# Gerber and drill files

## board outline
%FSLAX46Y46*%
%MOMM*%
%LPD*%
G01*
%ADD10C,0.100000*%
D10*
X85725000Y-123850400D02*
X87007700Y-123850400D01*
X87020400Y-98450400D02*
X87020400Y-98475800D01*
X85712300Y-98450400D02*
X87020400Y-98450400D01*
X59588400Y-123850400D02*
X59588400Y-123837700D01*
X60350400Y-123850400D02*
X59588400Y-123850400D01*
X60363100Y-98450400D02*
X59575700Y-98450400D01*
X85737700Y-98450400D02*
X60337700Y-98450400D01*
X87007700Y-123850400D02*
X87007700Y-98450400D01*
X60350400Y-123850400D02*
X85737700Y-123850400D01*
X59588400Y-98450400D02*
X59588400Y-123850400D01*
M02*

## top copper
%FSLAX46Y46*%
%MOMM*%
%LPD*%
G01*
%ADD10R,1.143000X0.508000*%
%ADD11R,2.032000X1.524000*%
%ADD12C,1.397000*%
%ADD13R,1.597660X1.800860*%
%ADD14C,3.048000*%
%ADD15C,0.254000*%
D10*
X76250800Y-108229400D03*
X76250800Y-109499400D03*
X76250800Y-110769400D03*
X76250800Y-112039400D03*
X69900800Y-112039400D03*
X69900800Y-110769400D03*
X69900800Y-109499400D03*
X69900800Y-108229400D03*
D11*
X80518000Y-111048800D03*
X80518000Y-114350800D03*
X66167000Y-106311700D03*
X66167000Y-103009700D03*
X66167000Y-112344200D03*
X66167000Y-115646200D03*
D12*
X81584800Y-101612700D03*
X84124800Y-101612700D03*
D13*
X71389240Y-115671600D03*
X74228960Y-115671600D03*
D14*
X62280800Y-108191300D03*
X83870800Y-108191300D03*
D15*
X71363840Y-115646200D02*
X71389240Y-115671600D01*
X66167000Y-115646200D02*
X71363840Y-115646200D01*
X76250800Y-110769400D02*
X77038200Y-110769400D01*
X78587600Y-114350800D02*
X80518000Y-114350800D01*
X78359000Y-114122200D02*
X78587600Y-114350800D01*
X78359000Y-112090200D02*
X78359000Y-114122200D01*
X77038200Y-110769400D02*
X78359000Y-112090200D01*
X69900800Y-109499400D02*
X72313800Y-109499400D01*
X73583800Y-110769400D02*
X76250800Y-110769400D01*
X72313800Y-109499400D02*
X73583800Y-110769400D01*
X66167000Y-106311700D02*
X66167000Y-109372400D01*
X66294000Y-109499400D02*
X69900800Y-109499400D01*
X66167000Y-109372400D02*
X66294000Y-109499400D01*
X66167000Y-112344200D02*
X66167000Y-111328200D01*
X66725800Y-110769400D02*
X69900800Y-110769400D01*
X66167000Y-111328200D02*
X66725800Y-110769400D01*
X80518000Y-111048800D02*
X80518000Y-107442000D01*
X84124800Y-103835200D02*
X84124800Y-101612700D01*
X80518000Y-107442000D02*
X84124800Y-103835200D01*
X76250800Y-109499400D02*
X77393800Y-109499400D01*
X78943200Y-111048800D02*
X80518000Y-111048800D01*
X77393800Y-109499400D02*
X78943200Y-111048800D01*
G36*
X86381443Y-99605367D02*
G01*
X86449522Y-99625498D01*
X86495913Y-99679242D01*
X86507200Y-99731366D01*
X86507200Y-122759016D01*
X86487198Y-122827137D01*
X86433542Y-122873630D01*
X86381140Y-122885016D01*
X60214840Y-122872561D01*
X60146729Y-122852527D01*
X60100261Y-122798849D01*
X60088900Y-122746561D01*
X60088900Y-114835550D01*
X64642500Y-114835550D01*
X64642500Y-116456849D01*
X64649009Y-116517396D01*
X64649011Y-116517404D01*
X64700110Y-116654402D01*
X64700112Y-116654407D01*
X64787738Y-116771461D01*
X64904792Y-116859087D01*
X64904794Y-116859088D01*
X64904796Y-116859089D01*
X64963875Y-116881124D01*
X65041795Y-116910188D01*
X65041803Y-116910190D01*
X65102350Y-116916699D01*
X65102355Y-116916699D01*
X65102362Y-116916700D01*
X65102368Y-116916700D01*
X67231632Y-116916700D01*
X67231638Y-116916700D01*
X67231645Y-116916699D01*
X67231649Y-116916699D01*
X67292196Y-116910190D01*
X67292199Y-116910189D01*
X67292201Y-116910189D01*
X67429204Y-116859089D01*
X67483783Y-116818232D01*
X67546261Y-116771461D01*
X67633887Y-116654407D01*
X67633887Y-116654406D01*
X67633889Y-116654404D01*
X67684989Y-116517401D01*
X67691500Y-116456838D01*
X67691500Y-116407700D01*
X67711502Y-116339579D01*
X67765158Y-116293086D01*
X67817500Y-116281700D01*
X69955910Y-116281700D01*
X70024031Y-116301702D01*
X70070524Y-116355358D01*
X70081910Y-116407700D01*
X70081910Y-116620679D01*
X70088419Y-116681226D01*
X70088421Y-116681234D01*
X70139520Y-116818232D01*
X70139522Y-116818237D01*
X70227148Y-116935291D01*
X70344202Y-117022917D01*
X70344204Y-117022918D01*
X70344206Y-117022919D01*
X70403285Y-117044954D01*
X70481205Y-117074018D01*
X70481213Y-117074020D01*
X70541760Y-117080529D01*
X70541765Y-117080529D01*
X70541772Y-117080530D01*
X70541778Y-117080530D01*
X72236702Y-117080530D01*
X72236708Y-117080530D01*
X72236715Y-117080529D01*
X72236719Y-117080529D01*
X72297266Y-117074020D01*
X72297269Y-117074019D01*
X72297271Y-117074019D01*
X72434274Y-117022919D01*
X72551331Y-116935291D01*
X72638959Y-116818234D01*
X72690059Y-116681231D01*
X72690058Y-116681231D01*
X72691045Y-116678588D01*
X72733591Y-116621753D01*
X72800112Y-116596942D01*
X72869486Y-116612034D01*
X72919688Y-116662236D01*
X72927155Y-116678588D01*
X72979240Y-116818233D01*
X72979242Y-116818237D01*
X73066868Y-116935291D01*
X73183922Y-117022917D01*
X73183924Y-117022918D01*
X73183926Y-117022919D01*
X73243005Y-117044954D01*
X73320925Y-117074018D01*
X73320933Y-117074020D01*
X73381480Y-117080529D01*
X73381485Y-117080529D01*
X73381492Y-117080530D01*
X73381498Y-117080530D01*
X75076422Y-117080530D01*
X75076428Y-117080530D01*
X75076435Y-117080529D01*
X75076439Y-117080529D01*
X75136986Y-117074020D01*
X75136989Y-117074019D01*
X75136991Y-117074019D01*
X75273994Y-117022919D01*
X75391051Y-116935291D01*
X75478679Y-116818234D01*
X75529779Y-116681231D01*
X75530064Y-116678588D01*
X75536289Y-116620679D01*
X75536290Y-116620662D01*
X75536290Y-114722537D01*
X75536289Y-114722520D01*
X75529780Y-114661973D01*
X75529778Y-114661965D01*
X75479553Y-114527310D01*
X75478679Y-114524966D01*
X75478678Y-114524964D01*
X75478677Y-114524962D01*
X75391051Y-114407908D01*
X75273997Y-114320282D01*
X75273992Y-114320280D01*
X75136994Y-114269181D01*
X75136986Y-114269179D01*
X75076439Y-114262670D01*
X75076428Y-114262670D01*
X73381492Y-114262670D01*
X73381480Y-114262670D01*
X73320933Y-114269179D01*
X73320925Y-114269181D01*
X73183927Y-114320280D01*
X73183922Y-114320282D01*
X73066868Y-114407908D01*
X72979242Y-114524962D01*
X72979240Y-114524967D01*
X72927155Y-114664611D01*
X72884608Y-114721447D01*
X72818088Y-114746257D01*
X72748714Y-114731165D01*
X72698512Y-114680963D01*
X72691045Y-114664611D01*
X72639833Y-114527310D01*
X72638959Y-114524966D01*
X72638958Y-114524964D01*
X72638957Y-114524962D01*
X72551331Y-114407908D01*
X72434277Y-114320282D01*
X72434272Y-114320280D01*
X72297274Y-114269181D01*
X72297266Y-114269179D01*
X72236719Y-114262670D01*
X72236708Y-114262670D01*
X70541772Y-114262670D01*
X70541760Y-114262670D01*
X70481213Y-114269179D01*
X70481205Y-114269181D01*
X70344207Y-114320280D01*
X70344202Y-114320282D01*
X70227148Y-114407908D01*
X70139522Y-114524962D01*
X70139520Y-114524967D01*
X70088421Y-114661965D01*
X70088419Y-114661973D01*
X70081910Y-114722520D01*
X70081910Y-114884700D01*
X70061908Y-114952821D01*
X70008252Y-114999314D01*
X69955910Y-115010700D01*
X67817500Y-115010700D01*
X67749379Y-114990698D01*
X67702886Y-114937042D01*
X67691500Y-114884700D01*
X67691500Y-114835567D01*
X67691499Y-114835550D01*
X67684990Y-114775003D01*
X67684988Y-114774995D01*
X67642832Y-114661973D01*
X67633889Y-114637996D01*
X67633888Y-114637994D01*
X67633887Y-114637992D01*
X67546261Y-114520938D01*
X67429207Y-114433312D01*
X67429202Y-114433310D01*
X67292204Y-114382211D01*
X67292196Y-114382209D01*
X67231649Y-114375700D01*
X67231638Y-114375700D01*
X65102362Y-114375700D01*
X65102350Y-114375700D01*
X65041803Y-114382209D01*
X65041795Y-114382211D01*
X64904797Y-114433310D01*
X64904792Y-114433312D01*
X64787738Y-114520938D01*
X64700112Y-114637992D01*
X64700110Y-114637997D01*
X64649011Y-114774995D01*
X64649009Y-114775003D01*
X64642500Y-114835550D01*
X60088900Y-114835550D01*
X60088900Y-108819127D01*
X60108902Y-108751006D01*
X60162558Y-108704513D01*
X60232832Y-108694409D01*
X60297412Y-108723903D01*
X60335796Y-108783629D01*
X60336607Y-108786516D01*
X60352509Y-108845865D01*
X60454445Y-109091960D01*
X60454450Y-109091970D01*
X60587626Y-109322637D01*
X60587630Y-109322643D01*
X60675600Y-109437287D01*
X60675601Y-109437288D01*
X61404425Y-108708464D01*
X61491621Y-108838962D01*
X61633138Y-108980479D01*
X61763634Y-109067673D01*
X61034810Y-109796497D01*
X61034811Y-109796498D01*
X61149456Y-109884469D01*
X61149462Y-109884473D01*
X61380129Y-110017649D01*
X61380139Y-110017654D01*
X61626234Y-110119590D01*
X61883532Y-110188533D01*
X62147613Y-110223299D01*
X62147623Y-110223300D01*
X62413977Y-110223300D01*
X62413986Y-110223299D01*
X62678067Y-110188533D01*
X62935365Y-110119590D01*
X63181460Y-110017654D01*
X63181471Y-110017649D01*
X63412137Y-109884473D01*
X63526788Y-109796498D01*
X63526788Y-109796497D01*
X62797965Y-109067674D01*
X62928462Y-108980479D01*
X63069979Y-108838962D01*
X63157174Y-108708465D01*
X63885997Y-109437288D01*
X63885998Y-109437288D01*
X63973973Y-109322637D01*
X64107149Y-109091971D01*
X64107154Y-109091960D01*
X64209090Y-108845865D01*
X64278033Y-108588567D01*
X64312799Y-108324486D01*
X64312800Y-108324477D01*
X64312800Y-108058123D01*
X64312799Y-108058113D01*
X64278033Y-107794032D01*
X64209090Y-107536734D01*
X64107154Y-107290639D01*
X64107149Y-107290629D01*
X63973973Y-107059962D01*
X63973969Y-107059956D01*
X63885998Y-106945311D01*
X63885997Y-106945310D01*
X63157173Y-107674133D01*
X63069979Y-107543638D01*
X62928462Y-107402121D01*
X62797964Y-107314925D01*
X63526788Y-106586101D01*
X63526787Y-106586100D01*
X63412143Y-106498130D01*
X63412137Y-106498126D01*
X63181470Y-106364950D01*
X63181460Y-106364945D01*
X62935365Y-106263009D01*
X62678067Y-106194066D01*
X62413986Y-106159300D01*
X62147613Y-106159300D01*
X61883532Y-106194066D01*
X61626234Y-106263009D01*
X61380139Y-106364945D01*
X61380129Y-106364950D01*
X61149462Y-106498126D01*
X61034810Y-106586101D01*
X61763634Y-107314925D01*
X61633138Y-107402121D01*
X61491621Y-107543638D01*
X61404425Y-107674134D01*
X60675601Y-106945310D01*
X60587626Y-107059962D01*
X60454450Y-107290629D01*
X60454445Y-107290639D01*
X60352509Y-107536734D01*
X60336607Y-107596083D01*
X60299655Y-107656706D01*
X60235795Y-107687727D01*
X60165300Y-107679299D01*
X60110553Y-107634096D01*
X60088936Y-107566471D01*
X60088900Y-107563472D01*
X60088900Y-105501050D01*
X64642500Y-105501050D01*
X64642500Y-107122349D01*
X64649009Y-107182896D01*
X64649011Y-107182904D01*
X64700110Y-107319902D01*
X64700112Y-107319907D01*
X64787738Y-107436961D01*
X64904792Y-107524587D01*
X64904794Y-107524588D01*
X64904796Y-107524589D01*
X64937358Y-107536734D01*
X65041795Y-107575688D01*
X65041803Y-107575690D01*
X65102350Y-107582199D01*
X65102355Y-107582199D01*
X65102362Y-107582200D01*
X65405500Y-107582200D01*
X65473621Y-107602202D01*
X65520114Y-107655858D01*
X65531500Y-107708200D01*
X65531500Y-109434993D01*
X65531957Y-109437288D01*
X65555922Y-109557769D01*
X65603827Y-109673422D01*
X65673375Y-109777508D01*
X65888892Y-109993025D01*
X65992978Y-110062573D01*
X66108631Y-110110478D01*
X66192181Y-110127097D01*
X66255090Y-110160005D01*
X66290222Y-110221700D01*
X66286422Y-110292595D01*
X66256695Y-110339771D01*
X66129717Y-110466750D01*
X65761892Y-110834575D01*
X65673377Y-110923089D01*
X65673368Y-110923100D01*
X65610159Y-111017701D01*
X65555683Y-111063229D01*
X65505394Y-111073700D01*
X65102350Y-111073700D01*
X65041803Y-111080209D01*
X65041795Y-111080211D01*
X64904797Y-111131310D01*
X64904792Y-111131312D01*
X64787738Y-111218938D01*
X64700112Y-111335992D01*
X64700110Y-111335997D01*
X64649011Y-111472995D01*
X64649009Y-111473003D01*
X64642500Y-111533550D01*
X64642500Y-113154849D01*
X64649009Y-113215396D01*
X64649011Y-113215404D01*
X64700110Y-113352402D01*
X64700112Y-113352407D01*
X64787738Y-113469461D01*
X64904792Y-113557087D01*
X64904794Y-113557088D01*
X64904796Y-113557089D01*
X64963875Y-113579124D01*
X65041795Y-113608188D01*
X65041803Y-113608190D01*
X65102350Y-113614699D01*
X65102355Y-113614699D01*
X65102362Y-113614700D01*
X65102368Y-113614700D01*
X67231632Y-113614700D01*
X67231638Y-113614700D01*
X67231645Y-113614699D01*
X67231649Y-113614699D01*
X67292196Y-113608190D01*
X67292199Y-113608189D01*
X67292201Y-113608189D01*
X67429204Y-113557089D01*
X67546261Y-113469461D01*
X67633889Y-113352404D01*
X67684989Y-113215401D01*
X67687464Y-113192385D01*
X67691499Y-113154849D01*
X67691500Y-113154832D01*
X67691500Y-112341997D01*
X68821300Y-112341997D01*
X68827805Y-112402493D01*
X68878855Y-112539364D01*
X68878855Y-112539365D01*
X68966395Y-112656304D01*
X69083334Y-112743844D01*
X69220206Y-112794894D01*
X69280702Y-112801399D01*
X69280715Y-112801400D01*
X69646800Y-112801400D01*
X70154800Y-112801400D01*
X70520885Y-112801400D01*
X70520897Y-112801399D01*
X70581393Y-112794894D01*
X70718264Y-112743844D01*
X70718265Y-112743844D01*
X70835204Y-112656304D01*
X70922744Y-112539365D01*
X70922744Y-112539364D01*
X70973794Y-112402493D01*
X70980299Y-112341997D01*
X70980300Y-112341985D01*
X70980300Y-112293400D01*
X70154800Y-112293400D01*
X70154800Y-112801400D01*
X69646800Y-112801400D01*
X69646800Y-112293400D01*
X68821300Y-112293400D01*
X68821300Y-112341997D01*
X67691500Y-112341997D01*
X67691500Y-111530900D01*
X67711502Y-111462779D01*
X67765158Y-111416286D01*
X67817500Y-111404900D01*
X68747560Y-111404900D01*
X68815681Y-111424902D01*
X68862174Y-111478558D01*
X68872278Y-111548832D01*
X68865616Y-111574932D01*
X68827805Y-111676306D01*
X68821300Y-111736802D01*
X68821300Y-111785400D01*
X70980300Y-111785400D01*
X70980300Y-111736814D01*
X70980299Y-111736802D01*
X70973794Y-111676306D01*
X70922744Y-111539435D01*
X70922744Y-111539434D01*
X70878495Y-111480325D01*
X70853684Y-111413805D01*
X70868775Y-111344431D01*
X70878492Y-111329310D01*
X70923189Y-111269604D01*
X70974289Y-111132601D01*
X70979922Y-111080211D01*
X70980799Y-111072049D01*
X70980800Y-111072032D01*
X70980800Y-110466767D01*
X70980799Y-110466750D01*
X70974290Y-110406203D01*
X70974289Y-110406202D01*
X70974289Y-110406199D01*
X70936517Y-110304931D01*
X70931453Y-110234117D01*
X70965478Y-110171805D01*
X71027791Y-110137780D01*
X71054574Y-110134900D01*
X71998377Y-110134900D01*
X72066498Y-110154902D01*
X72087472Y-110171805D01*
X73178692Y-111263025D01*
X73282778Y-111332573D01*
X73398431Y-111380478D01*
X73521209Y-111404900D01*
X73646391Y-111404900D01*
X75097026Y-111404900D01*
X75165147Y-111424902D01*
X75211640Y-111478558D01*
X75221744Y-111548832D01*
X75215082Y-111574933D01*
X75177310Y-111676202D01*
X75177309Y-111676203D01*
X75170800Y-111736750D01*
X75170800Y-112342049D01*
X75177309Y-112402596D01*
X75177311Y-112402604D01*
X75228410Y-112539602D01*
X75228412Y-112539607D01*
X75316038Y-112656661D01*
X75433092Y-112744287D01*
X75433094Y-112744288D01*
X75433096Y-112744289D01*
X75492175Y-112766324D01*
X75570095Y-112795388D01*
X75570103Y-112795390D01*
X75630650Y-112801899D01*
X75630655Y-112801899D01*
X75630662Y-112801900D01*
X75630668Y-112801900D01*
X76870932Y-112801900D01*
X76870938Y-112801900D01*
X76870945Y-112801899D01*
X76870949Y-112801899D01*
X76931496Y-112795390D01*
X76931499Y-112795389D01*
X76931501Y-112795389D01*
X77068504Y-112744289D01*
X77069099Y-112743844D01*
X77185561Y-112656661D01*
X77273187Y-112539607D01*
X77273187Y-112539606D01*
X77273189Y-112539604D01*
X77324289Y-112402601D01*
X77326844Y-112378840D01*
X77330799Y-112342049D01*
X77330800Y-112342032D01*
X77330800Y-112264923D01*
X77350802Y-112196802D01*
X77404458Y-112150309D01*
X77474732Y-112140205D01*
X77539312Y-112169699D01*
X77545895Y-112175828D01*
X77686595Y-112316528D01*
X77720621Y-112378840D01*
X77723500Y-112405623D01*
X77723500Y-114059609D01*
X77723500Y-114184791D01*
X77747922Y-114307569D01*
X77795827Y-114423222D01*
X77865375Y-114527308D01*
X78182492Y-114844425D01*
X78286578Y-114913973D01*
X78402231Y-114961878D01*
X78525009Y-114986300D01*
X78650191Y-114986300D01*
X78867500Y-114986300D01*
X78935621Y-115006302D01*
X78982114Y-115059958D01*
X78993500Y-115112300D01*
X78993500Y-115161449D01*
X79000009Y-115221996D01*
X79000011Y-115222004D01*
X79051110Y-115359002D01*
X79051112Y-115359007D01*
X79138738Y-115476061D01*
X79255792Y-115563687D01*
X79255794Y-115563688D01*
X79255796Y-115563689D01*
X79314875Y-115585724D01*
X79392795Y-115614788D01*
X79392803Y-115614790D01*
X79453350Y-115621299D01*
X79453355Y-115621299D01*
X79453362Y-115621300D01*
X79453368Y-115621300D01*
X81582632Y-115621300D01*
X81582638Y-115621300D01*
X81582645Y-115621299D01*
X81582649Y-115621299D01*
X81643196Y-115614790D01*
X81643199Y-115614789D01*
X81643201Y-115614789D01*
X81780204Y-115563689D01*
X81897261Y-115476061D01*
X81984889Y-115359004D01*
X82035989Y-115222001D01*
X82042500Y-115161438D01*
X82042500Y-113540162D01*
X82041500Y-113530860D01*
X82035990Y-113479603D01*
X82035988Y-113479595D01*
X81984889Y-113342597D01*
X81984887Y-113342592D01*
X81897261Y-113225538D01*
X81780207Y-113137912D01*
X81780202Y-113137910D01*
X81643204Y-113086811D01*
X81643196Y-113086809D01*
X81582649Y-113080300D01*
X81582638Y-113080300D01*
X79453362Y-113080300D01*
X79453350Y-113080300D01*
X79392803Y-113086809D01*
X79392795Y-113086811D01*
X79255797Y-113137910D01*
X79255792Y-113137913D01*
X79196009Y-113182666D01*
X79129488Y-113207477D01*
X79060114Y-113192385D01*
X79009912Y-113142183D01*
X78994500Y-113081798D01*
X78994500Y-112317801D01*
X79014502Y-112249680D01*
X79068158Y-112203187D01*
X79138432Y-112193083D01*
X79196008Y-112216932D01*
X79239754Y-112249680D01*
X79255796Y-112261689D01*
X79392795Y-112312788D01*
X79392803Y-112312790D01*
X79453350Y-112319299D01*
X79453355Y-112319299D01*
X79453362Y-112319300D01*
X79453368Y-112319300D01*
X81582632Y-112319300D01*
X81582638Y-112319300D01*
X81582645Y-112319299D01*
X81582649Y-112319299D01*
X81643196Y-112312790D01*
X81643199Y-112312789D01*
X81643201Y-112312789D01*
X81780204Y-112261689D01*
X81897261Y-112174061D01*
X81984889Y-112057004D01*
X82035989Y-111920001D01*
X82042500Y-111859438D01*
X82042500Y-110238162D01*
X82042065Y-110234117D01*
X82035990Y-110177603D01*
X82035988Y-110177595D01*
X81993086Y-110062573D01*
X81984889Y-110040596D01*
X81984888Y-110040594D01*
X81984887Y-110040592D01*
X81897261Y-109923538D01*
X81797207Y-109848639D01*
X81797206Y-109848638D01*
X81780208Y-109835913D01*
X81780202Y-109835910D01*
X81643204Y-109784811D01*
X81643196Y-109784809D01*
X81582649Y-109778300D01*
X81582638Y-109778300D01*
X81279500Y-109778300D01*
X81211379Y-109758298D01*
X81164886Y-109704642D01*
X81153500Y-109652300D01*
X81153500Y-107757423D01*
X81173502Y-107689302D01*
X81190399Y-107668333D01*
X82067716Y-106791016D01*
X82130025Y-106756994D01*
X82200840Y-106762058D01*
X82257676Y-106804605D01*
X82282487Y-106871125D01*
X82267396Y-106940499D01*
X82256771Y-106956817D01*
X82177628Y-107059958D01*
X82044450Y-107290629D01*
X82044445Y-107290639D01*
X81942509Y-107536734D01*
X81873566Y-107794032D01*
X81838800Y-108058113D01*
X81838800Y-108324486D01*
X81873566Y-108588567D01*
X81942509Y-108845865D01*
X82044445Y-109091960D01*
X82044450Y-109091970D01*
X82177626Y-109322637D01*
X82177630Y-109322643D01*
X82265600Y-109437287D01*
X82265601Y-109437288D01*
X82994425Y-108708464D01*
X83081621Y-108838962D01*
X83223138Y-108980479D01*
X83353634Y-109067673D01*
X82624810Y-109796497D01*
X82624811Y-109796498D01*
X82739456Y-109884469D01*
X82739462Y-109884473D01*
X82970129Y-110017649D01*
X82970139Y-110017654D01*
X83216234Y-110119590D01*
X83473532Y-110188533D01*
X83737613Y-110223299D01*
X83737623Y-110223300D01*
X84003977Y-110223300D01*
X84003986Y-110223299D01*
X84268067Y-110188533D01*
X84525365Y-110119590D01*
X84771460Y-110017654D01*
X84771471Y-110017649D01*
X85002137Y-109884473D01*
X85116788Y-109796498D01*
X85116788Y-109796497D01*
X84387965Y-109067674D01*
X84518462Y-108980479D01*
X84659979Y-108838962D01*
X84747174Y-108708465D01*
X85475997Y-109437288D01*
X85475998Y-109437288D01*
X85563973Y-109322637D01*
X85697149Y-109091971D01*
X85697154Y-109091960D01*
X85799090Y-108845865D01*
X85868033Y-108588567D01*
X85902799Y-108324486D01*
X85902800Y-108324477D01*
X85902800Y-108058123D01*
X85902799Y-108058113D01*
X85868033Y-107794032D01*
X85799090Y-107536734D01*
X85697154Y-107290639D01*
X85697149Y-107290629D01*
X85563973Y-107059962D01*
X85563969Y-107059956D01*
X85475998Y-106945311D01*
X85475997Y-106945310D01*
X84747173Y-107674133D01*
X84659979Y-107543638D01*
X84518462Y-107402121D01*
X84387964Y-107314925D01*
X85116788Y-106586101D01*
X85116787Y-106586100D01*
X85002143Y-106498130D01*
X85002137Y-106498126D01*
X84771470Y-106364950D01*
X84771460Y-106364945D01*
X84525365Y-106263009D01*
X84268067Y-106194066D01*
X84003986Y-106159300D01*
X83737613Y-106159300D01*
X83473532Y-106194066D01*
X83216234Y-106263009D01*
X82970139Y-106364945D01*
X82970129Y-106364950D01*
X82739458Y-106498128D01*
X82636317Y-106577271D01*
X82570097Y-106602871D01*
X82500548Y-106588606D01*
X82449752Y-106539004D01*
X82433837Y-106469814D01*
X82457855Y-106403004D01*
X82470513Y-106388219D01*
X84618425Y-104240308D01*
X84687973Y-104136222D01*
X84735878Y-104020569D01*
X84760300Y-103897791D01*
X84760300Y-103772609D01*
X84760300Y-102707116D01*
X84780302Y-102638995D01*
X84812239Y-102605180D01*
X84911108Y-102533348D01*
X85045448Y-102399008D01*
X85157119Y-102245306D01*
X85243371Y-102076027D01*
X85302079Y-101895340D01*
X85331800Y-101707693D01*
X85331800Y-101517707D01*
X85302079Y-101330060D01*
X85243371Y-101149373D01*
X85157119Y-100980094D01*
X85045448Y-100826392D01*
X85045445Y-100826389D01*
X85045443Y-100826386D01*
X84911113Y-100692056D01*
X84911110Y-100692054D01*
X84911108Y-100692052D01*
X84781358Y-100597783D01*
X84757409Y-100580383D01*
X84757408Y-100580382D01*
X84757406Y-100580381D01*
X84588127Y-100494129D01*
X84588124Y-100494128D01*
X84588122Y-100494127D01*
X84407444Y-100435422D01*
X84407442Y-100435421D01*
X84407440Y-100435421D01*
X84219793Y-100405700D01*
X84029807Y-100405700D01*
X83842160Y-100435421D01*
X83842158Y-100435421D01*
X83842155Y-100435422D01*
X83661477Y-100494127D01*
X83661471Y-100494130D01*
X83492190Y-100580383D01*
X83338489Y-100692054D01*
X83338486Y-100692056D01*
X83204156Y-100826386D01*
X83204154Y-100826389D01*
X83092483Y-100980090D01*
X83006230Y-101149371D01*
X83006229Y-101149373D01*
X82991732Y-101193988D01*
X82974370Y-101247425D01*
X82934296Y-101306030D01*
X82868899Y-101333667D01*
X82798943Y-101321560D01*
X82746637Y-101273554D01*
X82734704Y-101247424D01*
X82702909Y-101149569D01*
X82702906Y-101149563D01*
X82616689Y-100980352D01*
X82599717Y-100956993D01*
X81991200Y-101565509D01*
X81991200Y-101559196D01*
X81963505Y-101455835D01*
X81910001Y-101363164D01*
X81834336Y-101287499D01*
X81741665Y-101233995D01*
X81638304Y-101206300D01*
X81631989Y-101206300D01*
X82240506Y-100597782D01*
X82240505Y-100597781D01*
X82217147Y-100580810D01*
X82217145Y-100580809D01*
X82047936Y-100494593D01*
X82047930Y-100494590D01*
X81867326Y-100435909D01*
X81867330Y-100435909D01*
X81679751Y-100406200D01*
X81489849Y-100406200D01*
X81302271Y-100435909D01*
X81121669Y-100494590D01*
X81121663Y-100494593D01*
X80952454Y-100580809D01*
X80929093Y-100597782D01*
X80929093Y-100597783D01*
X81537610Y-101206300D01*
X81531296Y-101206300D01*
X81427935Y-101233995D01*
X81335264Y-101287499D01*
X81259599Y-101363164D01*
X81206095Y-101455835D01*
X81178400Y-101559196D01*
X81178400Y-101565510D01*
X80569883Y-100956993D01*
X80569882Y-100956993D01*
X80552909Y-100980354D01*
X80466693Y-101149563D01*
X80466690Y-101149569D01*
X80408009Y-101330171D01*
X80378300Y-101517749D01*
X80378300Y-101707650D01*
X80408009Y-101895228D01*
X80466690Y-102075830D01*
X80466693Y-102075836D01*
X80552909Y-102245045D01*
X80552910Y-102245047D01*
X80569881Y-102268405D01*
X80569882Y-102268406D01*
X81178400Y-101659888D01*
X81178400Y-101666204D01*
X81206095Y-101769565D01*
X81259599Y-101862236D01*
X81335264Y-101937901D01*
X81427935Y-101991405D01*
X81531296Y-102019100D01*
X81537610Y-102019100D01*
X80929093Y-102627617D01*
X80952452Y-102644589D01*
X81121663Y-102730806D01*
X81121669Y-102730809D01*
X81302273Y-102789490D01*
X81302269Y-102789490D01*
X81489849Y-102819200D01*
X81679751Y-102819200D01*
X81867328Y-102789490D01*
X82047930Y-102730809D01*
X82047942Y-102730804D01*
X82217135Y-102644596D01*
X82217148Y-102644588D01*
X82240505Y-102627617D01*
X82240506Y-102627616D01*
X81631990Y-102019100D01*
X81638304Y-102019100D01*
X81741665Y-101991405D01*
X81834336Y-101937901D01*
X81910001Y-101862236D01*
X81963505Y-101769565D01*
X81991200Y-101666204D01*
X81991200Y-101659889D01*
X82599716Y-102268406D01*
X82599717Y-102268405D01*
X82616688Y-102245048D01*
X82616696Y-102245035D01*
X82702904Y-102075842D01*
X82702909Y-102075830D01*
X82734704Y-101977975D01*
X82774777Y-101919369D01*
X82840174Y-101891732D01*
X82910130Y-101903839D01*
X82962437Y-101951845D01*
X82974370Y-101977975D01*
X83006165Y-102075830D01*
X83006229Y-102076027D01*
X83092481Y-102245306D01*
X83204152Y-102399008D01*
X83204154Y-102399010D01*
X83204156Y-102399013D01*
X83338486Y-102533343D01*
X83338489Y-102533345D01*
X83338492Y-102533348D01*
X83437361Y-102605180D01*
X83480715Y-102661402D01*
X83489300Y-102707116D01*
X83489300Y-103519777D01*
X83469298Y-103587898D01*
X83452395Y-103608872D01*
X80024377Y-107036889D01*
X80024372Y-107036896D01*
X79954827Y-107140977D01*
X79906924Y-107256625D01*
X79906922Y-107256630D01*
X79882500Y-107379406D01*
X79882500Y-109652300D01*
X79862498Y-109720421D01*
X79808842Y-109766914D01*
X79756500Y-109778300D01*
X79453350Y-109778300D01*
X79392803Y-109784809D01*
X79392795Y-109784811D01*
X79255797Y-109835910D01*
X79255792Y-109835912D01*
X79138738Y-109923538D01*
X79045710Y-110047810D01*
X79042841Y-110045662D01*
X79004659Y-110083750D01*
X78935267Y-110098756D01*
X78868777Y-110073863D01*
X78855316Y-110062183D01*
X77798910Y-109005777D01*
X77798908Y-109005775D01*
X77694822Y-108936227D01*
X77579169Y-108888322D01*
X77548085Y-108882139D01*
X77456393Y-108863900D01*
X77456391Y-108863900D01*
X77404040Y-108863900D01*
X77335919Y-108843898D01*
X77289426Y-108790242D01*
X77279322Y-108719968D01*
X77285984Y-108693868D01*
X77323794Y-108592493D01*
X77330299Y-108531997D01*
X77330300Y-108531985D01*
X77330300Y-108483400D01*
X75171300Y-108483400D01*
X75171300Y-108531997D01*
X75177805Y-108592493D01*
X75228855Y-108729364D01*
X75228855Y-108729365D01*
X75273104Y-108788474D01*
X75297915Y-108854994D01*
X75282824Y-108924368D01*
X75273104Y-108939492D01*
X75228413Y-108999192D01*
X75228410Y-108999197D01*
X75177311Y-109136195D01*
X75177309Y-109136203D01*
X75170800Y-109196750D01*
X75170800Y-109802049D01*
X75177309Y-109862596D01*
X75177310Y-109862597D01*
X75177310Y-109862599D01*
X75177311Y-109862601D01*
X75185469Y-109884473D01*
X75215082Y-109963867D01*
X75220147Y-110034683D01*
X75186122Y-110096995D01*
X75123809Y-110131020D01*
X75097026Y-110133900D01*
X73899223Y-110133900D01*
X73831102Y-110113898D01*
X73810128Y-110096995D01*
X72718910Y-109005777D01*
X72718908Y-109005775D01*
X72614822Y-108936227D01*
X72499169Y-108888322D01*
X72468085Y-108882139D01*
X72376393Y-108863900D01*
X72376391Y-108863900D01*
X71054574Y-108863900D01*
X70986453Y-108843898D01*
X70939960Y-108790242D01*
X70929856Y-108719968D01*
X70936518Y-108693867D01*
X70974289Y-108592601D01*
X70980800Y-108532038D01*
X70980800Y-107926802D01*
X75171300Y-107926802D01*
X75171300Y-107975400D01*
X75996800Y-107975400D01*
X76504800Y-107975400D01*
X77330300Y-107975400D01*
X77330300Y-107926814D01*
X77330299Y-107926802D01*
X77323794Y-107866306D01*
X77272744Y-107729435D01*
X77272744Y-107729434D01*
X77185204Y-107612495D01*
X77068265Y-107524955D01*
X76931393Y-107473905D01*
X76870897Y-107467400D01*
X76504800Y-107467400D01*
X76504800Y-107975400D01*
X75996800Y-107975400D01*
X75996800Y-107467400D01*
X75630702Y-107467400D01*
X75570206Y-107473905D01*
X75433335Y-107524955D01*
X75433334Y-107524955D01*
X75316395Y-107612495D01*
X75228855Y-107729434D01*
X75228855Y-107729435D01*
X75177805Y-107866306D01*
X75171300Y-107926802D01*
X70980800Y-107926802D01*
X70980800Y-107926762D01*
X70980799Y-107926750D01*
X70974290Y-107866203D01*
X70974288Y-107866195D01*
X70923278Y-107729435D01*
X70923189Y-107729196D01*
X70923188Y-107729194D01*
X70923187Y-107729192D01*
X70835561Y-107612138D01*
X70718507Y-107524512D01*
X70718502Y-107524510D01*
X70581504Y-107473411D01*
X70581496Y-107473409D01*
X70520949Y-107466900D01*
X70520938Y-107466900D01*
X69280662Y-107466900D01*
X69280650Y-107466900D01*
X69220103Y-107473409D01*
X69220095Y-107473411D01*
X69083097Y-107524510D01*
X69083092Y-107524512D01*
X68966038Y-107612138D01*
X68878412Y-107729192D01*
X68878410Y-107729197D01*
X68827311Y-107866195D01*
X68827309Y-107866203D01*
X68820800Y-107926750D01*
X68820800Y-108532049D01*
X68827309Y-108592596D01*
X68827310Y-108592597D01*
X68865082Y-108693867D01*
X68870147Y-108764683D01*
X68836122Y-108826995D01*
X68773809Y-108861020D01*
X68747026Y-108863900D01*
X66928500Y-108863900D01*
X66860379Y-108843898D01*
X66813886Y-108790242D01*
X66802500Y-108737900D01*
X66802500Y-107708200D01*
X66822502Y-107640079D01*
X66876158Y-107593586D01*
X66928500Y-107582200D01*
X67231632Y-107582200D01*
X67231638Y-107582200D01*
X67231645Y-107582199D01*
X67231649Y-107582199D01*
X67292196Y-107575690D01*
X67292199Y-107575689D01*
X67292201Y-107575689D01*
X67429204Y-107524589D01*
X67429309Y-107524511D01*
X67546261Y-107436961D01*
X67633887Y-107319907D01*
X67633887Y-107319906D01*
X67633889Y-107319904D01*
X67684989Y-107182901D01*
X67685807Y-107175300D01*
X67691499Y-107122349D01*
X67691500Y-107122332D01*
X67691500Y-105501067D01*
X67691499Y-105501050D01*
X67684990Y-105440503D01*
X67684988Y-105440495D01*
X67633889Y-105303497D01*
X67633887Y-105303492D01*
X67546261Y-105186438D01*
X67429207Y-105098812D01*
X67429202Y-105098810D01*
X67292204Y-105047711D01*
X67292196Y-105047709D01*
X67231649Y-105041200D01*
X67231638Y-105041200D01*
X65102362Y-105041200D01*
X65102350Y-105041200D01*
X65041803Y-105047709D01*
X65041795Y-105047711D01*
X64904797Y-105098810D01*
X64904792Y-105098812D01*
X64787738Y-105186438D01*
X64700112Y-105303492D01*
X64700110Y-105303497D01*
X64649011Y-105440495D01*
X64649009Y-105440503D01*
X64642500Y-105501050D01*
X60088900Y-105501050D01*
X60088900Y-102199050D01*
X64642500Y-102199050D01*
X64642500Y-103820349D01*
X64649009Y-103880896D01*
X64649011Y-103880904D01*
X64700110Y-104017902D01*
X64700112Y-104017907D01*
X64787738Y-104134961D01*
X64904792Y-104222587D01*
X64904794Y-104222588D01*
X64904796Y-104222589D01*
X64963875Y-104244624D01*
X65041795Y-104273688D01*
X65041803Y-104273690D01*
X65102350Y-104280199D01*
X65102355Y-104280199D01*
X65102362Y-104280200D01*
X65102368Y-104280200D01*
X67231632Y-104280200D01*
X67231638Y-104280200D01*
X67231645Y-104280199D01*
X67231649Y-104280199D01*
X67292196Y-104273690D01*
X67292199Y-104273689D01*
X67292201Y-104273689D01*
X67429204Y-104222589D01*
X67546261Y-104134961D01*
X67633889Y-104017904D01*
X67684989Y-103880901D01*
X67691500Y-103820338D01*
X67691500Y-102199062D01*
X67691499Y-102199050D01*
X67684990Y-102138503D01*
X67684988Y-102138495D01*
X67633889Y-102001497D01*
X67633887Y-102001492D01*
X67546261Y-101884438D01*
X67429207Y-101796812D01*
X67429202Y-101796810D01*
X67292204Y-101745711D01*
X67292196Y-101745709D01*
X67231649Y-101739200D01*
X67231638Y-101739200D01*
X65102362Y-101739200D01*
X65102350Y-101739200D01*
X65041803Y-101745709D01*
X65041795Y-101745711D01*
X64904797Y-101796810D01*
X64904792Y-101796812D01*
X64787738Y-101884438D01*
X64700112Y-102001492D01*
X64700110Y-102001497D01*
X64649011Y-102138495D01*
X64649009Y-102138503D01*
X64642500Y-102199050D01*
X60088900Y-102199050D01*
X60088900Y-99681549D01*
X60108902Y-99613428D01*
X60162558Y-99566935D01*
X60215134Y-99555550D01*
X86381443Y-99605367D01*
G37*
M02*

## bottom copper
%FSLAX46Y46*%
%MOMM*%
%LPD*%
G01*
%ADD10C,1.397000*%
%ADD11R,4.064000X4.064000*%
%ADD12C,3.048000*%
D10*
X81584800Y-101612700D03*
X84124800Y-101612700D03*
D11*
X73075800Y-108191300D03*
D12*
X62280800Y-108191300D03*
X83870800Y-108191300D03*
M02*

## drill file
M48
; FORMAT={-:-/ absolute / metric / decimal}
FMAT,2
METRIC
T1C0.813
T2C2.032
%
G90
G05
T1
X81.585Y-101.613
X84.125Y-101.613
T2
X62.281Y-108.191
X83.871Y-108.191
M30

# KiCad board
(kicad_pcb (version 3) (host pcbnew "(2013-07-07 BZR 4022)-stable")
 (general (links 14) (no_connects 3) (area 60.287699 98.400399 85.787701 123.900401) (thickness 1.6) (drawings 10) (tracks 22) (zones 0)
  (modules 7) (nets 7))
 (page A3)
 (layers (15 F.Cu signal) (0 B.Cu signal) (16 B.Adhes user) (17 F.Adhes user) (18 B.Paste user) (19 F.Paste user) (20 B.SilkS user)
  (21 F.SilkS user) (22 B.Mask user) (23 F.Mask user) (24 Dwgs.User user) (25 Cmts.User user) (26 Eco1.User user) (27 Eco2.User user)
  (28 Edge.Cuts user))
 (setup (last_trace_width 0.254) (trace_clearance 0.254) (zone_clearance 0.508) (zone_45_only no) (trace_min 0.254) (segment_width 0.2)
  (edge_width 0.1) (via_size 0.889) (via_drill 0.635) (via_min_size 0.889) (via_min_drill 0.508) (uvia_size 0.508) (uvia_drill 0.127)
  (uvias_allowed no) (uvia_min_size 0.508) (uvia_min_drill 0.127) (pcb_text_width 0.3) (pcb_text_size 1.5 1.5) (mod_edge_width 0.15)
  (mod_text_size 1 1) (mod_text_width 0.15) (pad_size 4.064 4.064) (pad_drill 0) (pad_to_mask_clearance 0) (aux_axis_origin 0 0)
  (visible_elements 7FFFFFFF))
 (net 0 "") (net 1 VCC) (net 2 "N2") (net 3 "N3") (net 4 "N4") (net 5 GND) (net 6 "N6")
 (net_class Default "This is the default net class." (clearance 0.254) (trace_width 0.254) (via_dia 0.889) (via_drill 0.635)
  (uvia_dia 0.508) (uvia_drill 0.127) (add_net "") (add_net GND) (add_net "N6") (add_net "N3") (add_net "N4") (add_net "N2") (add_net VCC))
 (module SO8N (layer F.Cu) (at 73.0758 110.1344 270)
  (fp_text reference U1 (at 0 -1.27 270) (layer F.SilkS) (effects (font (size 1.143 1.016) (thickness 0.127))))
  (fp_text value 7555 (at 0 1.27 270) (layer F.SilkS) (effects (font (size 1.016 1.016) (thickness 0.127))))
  (pad 8 smd rect (at -1.905 -3.175 270) (size 0.508 1.143) (layers F.Cu F.Paste F.Mask) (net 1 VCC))
  (pad 7 smd rect (at -0.635 -3.175 270) (size 0.508 1.143) (layers F.Cu F.Paste F.Mask) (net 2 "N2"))
  (pad 6 smd rect (at 0.635 -3.175 270) (size 0.508 1.143) (layers F.Cu F.Paste F.Mask) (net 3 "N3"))
  (pad 5 smd rect (at 1.905 -3.175 270) (size 0.508 1.143) (layers F.Cu F.Paste F.Mask))
  (pad 4 smd rect (at 1.905 3.175 270) (size 0.508 1.143) (layers F.Cu F.Paste F.Mask) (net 1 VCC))
  (pad 3 smd rect (at 0.635 3.175 270) (size 0.508 1.143) (layers F.Cu F.Paste F.Mask) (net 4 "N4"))
  (pad 2 smd rect (at -0.635 3.175 270) (size 0.508 1.143) (layers F.Cu F.Paste F.Mask) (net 3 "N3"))
  (pad 1 smd rect (at -1.905 3.175 270) (size 0.508 1.143) (layers F.Cu F.Paste F.Mask) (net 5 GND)))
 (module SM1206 (layer F.Cu) (at 80.518 112.6998 270)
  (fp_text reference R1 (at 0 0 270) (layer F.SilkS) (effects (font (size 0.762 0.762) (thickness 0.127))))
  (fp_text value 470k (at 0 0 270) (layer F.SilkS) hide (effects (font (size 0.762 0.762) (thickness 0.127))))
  (pad 1 smd rect (at -1.651 0 270) (size 1.524 2.032) (layers F.Cu F.Paste F.Mask) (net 2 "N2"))
  (pad 2 smd rect (at 1.651 0 270) (size 1.524 2.032) (layers F.Cu F.Paste F.Mask) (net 3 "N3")))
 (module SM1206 (layer F.Cu) (at 66.167 104.6607 90)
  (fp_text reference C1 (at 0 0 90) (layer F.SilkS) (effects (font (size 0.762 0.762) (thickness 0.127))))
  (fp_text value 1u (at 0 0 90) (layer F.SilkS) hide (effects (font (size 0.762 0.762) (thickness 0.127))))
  (pad 1 smd rect (at -1.651 0 90) (size 1.524 2.032) (layers F.Cu F.Paste F.Mask) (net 3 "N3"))
  (pad 2 smd rect (at 1.651 0 90) (size 1.524 2.032) (layers F.Cu F.Paste F.Mask) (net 5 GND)))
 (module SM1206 (layer F.Cu) (at 66.167 113.9952 270)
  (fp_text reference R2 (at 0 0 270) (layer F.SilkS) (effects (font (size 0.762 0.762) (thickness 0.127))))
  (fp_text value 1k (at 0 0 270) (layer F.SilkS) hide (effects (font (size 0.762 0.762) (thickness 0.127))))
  (pad 1 smd rect (at -1.651 0 270) (size 1.524 2.032) (layers F.Cu F.Paste F.Mask) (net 4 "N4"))
  (pad 2 smd rect (at 1.651 0 270) (size 1.524 2.032) (layers F.Cu F.Paste F.Mask) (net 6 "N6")))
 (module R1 (layer F.Cu) (at 82.8548 101.6127) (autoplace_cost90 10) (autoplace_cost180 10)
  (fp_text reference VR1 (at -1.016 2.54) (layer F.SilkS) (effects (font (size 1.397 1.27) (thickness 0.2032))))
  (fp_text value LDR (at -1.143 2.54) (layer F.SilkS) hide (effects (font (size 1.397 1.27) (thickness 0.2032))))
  (pad 1 thru_hole circle (at -1.27 0) (size 1.397 1.397) (drill 0.8128) (layers *.Cu *.Mask F.SilkS) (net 1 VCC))
  (pad 2 thru_hole circle (at 1.27 0) (size 1.397 1.397) (drill 0.8128) (layers *.Cu *.Mask F.SilkS) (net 2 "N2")))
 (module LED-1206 (layer F.Cu) (at 72.8091 115.6716)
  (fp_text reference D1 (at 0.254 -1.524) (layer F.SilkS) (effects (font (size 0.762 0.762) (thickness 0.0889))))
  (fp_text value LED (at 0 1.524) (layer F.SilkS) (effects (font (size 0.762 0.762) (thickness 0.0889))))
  (pad 1 smd rect (at -1.41986 0) (size 1.59766 1.80086) (layers F.Cu F.Paste F.Mask) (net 6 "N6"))
  (pad 2 smd rect (at 1.41986 0) (size 1.59766 1.80086) (layers F.Cu F.Paste F.Mask) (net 5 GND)))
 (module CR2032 (layer B.Cu) (at 73.0758 108.1913 180)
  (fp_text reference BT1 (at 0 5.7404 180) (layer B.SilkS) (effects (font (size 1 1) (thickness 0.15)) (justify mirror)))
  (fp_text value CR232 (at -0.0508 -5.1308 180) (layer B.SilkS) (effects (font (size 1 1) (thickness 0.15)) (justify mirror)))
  (pad 2 smd rect (at 0 0 180) (size 4.064 4.064) (layers B.Cu B.Paste B.Mask) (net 5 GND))
  (pad 1 thru_hole circle (at 10.795 0 180) (size 3.048 3.048) (drill 2.032) (layers *.Cu *.Mask B.SilkS) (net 1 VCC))
  (pad 1 thru_hole circle (at -10.795 0 180) (size 3.048 3.048) (drill 2.032) (layers *.Cu *.Mask B.SilkS) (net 1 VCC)))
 (gr_line (start 85.725 123.8504) (end 87.0077 123.8504) (angle 90) (layer Edge.Cuts) (width 0.1))
 (gr_line (start 87.0204 98.4504) (end 87.0204 98.4758) (angle 90) (layer Edge.Cuts) (width 0.1))
 (gr_line (start 85.7123 98.4504) (end 87.0204 98.4504) (angle 90) (layer Edge.Cuts) (width 0.1))
 (gr_line (start 59.5884 123.8504) (end 59.5884 123.8377) (angle 90) (layer Edge.Cuts) (width 0.1))
 (gr_line (start 60.3504 123.8504) (end 59.5884 123.8504) (angle 90) (layer Edge.Cuts) (width 0.1))
 (gr_line (start 60.3631 98.4504) (end 59.5757 98.4504) (angle 90) (layer Edge.Cuts) (width 0.1))
 (gr_line (start 85.7377 98.4504) (end 60.3377 98.4504) (angle 90) (layer Edge.Cuts) (width 0.1))
 (gr_line (start 87.0077 123.8504) (end 87.0077 98.4504) (angle 90) (layer Edge.Cuts) (width 0.1))
 (gr_line (start 60.3504 123.8504) (end 85.7377 123.8504) (angle 90) (layer Edge.Cuts) (width 0.1))
 (gr_line (start 59.5884 98.4504) (end 59.5884 123.8504) (angle 90) (layer Edge.Cuts) (width 0.1))
 (segment (start 71.36384 115.6462) (end 71.38924 115.6716) (width 0.254) (layer F.Cu) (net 6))
 (segment (start 66.167 115.6462) (end 71.36384 115.6462) (width 0.254) (layer F.Cu) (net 6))
 (segment (start 76.2508 110.7694) (end 77.0382 110.7694) (width 0.254) (layer F.Cu) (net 3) (status 400000))
 (segment (start 78.5876 114.3508) (end 80.518 114.3508) (width 0.254) (layer F.Cu) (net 3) (status 800000))
 (segment (start 78.359 114.1222) (end 78.5876 114.3508) (width 0.254) (layer F.Cu) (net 3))
 (segment (start 78.359 112.0902) (end 78.359 114.1222) (width 0.254) (layer F.Cu) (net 3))
 (segment (start 77.0382 110.7694) (end 78.359 112.0902) (width 0.254) (layer F.Cu) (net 3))
 (segment (start 69.9008 109.4994) (end 72.3138 109.4994) (width 0.254) (layer F.Cu) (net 3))
 (segment (start 73.5838 110.7694) (end 76.2508 110.7694) (width 0.254) (layer F.Cu) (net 3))
 (segment (start 72.3138 109.4994) (end 73.5838 110.7694) (width 0.254) (layer F.Cu) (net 3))
 (segment (start 66.167 106.3117) (end 66.167 109.3724) (width 0.254) (layer F.Cu) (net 3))
 (segment (start 66.294 109.4994) (end 69.9008 109.4994) (width 0.254) (layer F.Cu) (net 3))
 (segment (start 66.167 109.3724) (end 66.294 109.4994) (width 0.254) (layer F.Cu) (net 3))
 (segment (start 66.167 112.3442) (end 66.167 111.3282) (width 0.254) (layer F.Cu) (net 4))
 (segment (start 66.7258 110.7694) (end 69.9008 110.7694) (width 0.254) (layer F.Cu) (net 4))
 (segment (start 66.167 111.3282) (end 66.7258 110.7694) (width 0.254) (layer F.Cu) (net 4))
 (segment (start 80.518 111.0488) (end 80.518 107.442) (width 0.254) (layer F.Cu) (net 2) (status 400000))
 (segment (start 84.1248 103.8352) (end 84.1248 101.6127) (width 0.254) (layer F.Cu) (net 2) (status 800000))
 (segment (start 80.518 107.442) (end 84.1248 103.8352) (width 0.254) (layer F.Cu) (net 2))
 (segment (start 76.2508 109.4994) (end 77.3938 109.4994) (width 0.254) (layer F.Cu) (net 2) (status 400000))
 (segment (start 78.9432 111.0488) (end 80.518 111.0488) (width 0.254) (layer F.Cu) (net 2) (status 800000))
 (segment (start 77.3938 109.4994) (end 78.9432 111.0488) (width 0.254) (layer F.Cu) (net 2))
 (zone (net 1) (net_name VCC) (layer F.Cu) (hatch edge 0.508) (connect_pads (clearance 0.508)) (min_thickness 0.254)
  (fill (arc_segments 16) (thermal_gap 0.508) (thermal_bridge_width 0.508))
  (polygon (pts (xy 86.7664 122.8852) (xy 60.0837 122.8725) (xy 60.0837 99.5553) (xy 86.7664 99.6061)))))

